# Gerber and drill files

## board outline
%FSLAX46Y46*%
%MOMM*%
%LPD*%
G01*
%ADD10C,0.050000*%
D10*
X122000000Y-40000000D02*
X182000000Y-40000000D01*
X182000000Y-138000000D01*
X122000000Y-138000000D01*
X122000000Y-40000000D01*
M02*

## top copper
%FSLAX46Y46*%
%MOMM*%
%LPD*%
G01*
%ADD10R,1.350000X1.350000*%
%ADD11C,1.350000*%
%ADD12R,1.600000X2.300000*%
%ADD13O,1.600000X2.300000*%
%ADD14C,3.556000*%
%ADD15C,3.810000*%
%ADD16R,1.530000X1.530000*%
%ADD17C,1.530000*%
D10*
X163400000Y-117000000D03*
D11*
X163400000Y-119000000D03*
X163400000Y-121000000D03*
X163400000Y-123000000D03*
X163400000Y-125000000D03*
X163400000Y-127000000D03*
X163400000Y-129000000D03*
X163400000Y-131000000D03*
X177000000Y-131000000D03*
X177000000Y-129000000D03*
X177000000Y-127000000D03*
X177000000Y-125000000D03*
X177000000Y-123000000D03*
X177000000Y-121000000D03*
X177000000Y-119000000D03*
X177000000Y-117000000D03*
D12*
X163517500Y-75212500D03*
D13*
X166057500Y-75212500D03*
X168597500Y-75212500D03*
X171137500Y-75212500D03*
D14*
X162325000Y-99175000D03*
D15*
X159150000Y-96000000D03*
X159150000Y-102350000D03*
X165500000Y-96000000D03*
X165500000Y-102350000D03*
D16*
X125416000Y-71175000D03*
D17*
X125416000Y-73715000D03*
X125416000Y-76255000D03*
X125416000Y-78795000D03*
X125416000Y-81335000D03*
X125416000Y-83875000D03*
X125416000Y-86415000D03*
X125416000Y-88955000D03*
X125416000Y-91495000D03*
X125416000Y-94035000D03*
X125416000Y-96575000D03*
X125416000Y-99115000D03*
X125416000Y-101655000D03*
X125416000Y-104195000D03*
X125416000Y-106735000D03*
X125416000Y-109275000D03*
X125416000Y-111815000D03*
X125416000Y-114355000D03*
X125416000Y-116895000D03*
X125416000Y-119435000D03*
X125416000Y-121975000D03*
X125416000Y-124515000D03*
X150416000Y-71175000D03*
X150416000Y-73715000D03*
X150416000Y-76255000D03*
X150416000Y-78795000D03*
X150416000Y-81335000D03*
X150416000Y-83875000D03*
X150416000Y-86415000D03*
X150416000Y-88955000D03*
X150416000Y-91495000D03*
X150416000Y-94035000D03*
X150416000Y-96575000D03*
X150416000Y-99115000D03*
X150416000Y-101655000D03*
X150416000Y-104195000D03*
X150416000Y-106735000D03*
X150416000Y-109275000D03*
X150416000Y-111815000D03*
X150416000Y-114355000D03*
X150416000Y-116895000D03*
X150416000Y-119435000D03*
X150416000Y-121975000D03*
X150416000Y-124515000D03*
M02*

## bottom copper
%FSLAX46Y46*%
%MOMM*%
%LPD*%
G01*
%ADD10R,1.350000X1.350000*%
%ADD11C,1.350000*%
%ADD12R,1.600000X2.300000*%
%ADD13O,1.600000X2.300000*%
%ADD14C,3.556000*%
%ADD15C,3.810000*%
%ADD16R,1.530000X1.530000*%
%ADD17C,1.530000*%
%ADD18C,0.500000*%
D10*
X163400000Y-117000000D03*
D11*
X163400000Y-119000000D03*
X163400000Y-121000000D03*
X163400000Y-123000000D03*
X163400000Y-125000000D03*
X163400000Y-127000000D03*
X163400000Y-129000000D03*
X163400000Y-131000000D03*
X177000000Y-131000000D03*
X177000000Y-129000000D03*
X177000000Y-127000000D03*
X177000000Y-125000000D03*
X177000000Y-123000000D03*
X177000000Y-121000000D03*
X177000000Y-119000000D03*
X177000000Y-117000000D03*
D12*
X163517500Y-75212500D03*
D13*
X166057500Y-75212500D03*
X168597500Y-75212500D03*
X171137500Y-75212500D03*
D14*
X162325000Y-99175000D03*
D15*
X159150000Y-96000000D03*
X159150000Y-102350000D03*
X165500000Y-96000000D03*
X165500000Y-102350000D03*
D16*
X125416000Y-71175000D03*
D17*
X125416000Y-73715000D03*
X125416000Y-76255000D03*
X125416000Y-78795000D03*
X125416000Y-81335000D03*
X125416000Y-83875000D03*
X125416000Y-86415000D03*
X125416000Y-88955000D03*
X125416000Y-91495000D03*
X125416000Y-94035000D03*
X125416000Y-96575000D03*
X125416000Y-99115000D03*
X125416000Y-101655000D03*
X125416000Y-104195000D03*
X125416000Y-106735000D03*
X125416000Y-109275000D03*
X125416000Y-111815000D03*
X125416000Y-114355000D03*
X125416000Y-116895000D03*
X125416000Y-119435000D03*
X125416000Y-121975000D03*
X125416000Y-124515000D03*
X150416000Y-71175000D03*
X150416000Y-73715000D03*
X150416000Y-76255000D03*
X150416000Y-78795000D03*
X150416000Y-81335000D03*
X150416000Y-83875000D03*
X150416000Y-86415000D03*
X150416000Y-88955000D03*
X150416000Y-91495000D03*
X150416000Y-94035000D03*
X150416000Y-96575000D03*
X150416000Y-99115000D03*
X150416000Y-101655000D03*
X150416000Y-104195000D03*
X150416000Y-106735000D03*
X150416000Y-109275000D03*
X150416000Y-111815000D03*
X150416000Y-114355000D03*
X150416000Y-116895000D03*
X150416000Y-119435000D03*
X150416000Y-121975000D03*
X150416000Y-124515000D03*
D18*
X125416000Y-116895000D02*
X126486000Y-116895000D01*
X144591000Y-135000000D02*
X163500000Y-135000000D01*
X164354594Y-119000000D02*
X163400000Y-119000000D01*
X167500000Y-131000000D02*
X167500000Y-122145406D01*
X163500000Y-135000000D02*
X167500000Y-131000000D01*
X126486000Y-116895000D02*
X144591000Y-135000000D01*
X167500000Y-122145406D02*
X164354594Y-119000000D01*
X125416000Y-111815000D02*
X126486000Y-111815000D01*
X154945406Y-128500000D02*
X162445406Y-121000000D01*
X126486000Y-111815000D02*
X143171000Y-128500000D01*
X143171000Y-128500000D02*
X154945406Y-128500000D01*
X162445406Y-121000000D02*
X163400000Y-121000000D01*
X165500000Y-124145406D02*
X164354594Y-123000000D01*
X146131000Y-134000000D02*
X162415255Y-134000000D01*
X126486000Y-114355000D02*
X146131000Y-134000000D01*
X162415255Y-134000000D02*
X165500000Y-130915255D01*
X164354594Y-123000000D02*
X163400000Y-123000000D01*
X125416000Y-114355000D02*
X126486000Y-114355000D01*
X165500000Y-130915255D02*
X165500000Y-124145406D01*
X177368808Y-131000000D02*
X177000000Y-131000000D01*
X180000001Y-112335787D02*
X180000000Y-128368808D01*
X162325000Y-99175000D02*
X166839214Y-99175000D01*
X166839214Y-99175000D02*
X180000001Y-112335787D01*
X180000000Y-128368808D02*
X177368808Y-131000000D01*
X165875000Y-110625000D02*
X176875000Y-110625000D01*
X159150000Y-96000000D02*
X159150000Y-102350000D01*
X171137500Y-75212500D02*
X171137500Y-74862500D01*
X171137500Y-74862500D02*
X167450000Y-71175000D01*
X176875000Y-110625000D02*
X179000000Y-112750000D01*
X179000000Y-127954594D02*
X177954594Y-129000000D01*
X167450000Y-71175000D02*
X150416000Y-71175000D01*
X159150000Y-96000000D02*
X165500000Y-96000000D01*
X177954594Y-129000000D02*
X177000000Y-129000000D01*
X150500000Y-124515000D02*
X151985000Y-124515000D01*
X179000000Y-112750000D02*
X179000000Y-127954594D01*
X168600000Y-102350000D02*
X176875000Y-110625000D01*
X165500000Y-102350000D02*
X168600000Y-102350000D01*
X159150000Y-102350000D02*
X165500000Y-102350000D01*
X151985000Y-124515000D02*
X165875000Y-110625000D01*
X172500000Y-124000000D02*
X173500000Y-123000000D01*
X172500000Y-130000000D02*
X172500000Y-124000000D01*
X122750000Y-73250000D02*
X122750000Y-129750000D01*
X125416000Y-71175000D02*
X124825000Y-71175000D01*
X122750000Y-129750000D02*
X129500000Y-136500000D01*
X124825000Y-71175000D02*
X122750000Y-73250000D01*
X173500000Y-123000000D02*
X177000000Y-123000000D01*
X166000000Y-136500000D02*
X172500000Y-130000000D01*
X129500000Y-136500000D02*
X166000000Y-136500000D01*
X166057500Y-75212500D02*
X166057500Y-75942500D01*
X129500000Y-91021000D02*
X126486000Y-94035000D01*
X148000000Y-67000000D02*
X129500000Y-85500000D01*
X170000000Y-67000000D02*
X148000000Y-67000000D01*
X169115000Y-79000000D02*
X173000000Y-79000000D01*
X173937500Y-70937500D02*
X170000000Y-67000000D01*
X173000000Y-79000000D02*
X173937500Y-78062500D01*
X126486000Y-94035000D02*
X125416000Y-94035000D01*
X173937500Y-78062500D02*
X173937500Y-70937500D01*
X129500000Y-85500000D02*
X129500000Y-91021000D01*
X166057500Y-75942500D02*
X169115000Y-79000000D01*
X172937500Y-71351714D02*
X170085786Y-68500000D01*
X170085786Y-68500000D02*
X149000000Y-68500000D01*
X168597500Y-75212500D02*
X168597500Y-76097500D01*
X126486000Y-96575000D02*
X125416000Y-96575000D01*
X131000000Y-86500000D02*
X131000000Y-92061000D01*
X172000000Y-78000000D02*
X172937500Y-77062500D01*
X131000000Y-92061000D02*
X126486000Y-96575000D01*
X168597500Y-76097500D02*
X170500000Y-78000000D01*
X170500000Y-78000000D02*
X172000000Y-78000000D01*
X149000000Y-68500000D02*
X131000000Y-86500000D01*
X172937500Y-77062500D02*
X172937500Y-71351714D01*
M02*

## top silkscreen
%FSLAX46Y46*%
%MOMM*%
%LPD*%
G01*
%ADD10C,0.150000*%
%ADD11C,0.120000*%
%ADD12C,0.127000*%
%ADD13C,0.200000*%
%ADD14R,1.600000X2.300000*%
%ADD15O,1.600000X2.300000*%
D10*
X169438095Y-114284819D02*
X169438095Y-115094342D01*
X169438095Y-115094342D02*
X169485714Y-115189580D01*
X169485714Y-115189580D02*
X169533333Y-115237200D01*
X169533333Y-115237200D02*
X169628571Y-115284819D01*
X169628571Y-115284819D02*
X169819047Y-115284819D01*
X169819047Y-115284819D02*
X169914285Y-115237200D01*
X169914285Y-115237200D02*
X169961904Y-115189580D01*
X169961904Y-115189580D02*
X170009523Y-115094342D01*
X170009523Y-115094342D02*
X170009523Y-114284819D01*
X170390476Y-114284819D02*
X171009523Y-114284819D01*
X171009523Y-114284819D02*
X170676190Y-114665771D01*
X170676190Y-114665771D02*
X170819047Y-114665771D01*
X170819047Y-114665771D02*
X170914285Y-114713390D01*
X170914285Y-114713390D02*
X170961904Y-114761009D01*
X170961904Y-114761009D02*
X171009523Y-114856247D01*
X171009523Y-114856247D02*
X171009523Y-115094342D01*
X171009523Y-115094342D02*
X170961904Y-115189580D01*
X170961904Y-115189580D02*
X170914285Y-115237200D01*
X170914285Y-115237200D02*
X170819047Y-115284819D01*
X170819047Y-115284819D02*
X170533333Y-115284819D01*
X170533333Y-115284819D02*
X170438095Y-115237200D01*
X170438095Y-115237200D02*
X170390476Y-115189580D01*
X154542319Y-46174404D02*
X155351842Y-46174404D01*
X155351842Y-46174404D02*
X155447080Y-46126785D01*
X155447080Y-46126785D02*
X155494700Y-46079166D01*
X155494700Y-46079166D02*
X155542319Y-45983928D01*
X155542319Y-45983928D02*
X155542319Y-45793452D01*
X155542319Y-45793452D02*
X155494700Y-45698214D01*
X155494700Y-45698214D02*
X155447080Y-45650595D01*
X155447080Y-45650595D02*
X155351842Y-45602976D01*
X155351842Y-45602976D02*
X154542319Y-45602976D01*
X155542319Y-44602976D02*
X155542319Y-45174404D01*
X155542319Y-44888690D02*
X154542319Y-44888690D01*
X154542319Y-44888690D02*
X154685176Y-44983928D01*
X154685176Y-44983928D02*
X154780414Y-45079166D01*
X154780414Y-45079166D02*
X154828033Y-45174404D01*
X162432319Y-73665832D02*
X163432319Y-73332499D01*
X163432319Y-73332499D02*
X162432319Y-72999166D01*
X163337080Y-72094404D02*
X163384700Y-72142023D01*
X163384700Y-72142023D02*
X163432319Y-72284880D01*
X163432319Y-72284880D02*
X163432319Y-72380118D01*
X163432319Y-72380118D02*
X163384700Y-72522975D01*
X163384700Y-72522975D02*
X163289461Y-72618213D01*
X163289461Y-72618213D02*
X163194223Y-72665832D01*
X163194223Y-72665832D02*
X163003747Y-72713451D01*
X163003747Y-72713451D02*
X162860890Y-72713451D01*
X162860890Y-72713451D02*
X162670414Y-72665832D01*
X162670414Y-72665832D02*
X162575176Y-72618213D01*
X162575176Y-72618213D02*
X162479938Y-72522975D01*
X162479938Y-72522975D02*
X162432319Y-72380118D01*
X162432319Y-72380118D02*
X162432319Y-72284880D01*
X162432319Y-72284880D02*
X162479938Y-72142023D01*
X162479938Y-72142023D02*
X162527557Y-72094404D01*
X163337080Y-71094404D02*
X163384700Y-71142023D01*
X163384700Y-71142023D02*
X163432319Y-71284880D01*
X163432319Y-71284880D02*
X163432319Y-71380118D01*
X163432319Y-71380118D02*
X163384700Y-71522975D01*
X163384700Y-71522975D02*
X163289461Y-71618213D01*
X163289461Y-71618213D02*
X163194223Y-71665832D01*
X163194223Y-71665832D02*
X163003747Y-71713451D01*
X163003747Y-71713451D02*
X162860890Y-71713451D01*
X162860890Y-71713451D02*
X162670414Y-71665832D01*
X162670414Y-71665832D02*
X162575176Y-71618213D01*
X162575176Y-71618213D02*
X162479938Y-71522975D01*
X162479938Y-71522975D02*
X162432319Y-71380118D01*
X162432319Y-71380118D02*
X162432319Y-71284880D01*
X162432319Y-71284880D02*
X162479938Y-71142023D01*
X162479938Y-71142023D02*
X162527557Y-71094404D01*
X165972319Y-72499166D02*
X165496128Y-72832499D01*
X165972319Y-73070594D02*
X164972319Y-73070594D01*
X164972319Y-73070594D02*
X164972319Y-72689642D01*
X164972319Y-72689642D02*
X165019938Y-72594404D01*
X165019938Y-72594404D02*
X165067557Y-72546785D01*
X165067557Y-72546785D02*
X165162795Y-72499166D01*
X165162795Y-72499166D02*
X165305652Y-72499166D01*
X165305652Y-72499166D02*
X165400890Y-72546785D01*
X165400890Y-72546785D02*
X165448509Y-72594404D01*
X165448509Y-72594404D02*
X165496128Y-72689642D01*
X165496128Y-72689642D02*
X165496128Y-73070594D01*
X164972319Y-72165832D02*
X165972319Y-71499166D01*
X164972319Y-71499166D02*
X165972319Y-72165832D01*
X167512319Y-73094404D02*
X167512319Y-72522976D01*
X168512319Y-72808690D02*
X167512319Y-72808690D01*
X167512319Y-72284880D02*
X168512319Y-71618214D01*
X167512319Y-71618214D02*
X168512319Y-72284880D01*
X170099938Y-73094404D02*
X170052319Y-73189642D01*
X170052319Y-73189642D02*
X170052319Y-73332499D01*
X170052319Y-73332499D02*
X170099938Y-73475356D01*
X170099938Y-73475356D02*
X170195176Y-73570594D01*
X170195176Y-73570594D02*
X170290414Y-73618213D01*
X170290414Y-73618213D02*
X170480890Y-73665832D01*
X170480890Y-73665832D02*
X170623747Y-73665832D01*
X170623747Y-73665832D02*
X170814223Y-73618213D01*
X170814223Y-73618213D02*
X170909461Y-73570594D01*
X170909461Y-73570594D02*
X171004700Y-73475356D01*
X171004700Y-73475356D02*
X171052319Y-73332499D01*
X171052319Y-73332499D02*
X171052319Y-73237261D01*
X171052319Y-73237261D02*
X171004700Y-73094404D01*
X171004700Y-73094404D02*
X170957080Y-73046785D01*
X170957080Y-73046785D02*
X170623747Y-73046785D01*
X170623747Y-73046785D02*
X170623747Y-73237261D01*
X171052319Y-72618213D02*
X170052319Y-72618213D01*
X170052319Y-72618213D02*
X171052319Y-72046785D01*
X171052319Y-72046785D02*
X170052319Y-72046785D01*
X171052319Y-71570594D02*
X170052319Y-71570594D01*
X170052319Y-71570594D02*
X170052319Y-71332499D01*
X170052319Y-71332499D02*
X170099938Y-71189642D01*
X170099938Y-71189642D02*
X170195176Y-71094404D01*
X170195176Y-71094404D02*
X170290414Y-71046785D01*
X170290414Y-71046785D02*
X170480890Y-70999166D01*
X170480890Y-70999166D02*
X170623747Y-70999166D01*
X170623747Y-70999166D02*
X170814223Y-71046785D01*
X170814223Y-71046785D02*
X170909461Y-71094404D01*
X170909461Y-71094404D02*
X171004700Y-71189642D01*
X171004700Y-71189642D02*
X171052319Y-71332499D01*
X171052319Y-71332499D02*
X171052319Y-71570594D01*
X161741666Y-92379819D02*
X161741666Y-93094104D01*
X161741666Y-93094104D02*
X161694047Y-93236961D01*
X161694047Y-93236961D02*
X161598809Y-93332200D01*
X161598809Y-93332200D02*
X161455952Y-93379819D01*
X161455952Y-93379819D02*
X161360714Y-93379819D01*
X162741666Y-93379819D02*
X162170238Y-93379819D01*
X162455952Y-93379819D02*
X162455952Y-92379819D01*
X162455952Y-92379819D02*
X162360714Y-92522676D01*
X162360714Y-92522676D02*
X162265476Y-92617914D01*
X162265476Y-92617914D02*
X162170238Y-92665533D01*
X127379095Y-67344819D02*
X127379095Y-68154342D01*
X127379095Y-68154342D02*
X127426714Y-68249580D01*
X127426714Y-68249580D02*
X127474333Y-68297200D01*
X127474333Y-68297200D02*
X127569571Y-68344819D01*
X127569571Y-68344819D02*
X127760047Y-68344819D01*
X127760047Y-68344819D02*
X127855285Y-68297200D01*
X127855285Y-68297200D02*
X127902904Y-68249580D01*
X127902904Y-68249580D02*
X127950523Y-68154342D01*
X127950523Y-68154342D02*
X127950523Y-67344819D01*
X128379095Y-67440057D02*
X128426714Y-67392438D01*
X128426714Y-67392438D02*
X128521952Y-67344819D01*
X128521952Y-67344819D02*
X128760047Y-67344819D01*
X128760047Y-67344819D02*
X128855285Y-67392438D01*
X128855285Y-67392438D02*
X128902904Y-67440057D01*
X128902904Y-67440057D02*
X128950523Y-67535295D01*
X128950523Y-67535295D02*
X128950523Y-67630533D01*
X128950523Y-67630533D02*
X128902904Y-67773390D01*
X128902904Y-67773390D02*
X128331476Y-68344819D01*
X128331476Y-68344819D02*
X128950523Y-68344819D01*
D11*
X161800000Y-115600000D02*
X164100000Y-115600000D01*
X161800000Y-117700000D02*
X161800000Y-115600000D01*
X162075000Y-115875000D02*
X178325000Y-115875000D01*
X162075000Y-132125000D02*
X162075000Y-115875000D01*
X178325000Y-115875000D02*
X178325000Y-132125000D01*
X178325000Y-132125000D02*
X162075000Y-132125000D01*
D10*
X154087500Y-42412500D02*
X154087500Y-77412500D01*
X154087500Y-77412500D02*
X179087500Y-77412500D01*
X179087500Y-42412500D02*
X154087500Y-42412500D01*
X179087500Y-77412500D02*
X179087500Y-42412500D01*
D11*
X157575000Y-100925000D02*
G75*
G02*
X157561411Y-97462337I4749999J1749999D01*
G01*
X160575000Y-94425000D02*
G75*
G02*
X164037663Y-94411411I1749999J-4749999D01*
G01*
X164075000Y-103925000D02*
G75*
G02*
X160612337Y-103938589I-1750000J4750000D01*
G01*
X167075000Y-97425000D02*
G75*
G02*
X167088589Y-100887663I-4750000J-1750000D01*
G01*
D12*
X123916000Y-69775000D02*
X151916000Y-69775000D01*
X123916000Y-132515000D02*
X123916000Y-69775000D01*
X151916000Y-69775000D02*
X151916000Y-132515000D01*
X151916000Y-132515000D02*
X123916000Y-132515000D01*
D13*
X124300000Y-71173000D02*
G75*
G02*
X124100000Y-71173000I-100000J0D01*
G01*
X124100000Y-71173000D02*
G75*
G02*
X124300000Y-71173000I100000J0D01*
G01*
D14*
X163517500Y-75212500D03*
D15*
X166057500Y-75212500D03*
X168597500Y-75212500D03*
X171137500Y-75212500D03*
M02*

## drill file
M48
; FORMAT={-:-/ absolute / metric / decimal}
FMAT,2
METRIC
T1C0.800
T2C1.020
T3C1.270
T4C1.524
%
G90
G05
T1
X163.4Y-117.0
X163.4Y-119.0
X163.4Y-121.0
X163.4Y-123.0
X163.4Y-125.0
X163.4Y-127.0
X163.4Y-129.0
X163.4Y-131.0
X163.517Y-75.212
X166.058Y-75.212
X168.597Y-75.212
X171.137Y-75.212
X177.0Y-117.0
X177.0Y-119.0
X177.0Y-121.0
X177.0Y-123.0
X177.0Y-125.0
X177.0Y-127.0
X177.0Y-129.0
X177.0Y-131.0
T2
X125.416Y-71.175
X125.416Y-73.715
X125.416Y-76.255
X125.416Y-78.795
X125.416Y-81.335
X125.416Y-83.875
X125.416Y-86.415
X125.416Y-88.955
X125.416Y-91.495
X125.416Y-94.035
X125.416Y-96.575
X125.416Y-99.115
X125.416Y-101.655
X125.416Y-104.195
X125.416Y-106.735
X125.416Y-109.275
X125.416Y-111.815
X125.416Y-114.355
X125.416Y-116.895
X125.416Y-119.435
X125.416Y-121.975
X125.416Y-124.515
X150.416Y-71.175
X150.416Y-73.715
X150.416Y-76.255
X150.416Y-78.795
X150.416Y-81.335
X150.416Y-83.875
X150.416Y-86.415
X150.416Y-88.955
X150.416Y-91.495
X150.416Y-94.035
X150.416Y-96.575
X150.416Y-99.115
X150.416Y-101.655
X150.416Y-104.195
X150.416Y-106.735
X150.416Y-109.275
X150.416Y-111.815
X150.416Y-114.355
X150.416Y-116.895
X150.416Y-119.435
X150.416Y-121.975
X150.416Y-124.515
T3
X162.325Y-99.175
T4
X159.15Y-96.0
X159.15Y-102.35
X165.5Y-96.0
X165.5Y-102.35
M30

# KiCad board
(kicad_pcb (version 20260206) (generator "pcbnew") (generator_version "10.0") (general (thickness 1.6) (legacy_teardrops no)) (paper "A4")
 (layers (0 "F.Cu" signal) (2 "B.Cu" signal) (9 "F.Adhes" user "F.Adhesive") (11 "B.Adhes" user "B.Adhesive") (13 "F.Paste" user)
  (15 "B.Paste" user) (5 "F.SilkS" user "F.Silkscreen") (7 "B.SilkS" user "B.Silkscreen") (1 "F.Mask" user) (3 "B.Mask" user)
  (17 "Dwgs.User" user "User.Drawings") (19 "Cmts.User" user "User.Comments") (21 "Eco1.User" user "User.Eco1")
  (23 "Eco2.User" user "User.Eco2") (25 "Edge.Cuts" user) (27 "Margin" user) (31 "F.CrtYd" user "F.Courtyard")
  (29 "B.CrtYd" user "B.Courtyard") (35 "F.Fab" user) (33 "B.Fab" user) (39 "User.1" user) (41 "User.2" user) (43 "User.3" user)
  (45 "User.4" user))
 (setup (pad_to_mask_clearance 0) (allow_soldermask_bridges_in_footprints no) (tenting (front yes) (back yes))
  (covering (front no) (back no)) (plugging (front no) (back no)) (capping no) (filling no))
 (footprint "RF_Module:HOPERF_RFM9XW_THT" (layer "F.Cu") (at 163.4 117)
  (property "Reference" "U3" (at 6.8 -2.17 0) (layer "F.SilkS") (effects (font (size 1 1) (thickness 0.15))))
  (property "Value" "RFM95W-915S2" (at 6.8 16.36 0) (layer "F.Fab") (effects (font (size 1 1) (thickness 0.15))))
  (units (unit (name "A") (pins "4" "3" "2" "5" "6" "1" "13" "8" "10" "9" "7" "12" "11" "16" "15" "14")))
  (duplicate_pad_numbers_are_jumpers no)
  (fp_line (start -1.6 -1.4) (end 0.7 -1.4) (stroke (width 0.12) (type solid)) (layer "F.SilkS"))
  (fp_line (start -1.6 0.7) (end -1.6 -1.4) (stroke (width 0.12) (type solid)) (layer "F.SilkS"))
  (fp_line (start -1.325 -1.125) (end 14.925 -1.125) (stroke (width 0.12) (type solid)) (layer "F.SilkS"))
  (fp_line (start -1.325 15.125) (end -1.325 -1.125) (stroke (width 0.12) (type solid)) (layer "F.SilkS"))
  (fp_line (start 14.925 -1.125) (end 14.925 15.125) (stroke (width 0.12) (type solid)) (layer "F.SilkS"))
  (fp_line (start 14.925 15.125) (end -1.325 15.125) (stroke (width 0.12) (type solid)) (layer "F.SilkS"))
  (pad "1" thru_hole rect (at 0 0) (size 1.35 1.35) (drill 0.8) (layers "*.Cu" "*.Mask") (remove_unused_layers no)
   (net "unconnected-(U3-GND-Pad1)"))
  (pad "2" thru_hole circle (at 0 2) (size 1.35 1.35) (drill 0.8) (layers "*.Cu" "*.Mask") (remove_unused_layers no) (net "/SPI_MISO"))
  (pad "3" thru_hole circle (at 0 4) (size 1.35 1.35) (drill 0.8) (layers "*.Cu" "*.Mask") (remove_unused_layers no) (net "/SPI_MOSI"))
  (pad "4" thru_hole circle (at 0 6) (size 1.35 1.35) (drill 0.8) (layers "*.Cu" "*.Mask") (remove_unused_layers no) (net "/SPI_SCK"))
  (pad "5" thru_hole circle (at 0 8) (size 1.35 1.35) (drill 0.8) (layers "*.Cu" "*.Mask") (remove_unused_layers no) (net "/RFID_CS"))
  (pad "6" thru_hole circle (at 0 10) (size 1.35 1.35) (drill 0.8) (layers "*.Cu" "*.Mask") (remove_unused_layers no) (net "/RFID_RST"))
  (pad "7" thru_hole circle (at 0 12) (size 1.35 1.35) (drill 0.8) (layers "*.Cu" "*.Mask") (remove_unused_layers no)
   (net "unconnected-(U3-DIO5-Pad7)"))
  (pad "8" thru_hole circle (at 0 14) (size 1.35 1.35) (drill 0.8) (layers "*.Cu" "*.Mask") (remove_unused_layers no)
   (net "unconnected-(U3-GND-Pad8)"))
  (pad "9" thru_hole circle (at 13.6 14) (size 1.35 1.35) (drill 0.8) (layers "*.Cu" "*.Mask") (remove_unused_layers no) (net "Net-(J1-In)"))
  (pad "10" thru_hole circle (at 13.6 12) (size 1.35 1.35) (drill 0.8) (layers "*.Cu" "*.Mask") (remove_unused_layers no)
   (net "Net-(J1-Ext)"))
  (pad "11" thru_hole circle (at 13.6 10) (size 1.35 1.35) (drill 0.8) (layers "*.Cu" "*.Mask") (remove_unused_layers no)
   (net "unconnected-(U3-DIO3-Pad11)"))
  (pad "12" thru_hole circle (at 13.6 8) (size 1.35 1.35) (drill 0.8) (layers "*.Cu" "*.Mask") (remove_unused_layers no)
   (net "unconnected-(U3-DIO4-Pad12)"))
  (pad "13" thru_hole circle (at 13.6 6) (size 1.35 1.35) (drill 0.8) (layers "*.Cu" "*.Mask") (remove_unused_layers no)
   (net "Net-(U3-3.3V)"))
  (pad "14" thru_hole circle (at 13.6 4) (size 1.35 1.35) (drill 0.8) (layers "*.Cu" "*.Mask") (remove_unused_layers no)
   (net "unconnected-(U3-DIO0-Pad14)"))
  (pad "15" thru_hole circle (at 13.6 2) (size 1.35 1.35) (drill 0.8) (layers "*.Cu" "*.Mask") (remove_unused_layers no)
   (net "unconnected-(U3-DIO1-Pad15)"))
  (pad "16" thru_hole circle (at 13.6 0) (size 1.35 1.35) (drill 0.8) (layers "*.Cu" "*.Mask") (remove_unused_layers no)
   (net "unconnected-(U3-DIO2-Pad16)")))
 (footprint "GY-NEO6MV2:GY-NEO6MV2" (layer "F.Cu") (at 154.0875 77.4125 -90)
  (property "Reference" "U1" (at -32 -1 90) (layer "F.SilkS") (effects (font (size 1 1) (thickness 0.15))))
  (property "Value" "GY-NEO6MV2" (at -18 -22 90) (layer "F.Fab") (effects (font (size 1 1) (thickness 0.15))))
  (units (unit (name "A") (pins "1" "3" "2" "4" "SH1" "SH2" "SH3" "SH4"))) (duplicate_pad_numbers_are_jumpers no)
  (fp_line (start -35 0) (end 0 0) (stroke (width 0.15) (type solid)) (layer "F.SilkS"))
  (fp_line (start 0 0) (end 0 -25) (stroke (width 0.15) (type solid)) (layer "F.SilkS"))
  (fp_line (start -35 -25) (end -35 0) (stroke (width 0.15) (type solid)) (layer "F.SilkS"))
  (fp_line (start 0 -25) (end -35 -25) (stroke (width 0.15) (type solid)) (layer "F.SilkS"))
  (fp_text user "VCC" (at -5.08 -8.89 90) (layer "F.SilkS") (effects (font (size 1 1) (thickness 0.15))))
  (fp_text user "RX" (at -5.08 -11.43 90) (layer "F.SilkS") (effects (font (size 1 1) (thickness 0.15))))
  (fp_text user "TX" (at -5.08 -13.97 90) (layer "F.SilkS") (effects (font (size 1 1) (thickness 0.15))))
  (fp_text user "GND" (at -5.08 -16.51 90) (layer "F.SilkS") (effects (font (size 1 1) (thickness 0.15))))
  (pad "1" thru_hole rect (at -2.2 -9.43 270) (size 2.3 1.6) (drill 0.8) (layers "*.Cu" "*.Mask" "F.SilkS") (remove_unused_layers no)
   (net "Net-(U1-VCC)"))
  (pad "2" thru_hole oval (at -2.2 -11.97 270) (size 2.3 1.6) (drill 0.8) (layers "*.Cu" "*.Mask" "F.SilkS") (remove_unused_layers no)
   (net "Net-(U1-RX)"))
  (pad "3" thru_hole oval (at -2.2 -14.51 270) (size 2.3 1.6) (drill 0.8) (layers "*.Cu" "*.Mask" "F.SilkS") (remove_unused_layers no)
   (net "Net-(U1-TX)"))
  (pad "4" thru_hole oval (at -2.2 -17.05 270) (size 2.3 1.6) (drill 0.8) (layers "*.Cu" "*.Mask" "F.SilkS") (remove_unused_layers no)
   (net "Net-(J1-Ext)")))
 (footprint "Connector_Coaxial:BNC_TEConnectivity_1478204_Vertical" (layer "F.Cu") (at 162.325 99.175)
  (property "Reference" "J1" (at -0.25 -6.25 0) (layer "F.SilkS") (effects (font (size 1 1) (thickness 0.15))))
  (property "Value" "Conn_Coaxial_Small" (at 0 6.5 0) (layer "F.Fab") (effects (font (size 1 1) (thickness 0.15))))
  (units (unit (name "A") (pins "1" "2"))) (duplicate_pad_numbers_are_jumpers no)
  (fp_arc (start -4.75 1.75) (mid -5.062075 0.019867) (end -4.763589 -1.712663) (stroke (width 0.12) (type solid)) (layer "F.SilkS"))
  (fp_arc (start -1.75 -4.75) (mid -0.019867 -5.062075) (end 1.712663 -4.763589) (stroke (width 0.12) (type solid)) (layer "F.SilkS"))
  (fp_arc (start 1.75 4.75) (mid 0.019867 5.062075) (end -1.712663 4.763589) (stroke (width 0.12) (type solid)) (layer "F.SilkS"))
  (fp_arc (start 4.75 -1.75) (mid 5.062075 -0.019867) (end 4.763589 1.712663) (stroke (width 0.12) (type solid)) (layer "F.SilkS"))
  (pad "1" thru_hole circle (at 0 0) (size 3.556 3.556) (drill 1.27) (layers "*.Cu" "*.Mask") (remove_unused_layers no) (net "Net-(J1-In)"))
  (pad "2" thru_hole circle (at -3.175 -3.175) (size 3.81 3.81) (drill 1.524) (layers "*.Cu" "*.Mask") (remove_unused_layers no)
   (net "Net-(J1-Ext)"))
  (pad "2" thru_hole circle (at -3.175 3.175) (size 3.81 3.81) (drill 1.524) (layers "*.Cu" "*.Mask") (remove_unused_layers no)
   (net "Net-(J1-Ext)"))
  (pad "2" thru_hole circle (at 3.175 -3.175) (size 3.81 3.81) (drill 1.524) (layers "*.Cu" "*.Mask") (remove_unused_layers no)
   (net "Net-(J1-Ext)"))
  (pad "2" thru_hole circle (at 3.175 3.175) (size 3.81 3.81) (drill 1.524) (layers "*.Cu" "*.Mask") (remove_unused_layers no)
   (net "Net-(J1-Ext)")))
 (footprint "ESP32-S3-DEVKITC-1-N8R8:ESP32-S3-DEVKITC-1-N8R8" (layer "F.Cu") (at 137.916 101.145)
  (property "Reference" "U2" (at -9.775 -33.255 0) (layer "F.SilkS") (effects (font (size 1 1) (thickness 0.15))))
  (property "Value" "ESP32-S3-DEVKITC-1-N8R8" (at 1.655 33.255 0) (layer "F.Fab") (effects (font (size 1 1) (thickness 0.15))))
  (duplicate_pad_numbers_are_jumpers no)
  (fp_line (start -14 -31.37) (end 14 -31.37) (stroke (width 0.127) (type solid)) (layer "F.SilkS"))
  (fp_line (start -14 31.37) (end -14 -31.37) (stroke (width 0.127) (type solid)) (layer "F.SilkS"))
  (fp_line (start 14 -31.37) (end 14 31.37) (stroke (width 0.127) (type solid)) (layer "F.SilkS"))
  (fp_line (start 14 31.37) (end -14 31.37) (stroke (width 0.127) (type solid)) (layer "F.SilkS"))
  (fp_circle (center -13.716 -29.972) (end -13.616 -29.972) (stroke (width 0.2) (type solid)) (fill no) (layer "F.SilkS"))
  (pad "J1_1" thru_hole rect (at -12.5 -29.97) (size 1.53 1.53) (drill 1.02) (layers "*.Cu" "*.Mask") (remove_unused_layers no)
   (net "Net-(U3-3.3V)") (solder_mask_margin 0.102))
  (pad "J1_2" thru_hole circle (at -12.5 -27.43) (size 1.53 1.53) (drill 1.02) (layers "*.Cu" "*.Mask") (remove_unused_layers no)
   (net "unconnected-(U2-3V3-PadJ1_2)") (solder_mask_margin 0.102))
  (pad "J1_3" thru_hole circle (at -12.5 -24.89) (size 1.53 1.53) (drill 1.02) (layers "*.Cu" "*.Mask") (remove_unused_layers no)
   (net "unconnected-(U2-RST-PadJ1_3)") (solder_mask_margin 0.102))
  (pad "J1_4" thru_hole circle (at -12.5 -22.35) (size 1.53 1.53) (drill 1.02) (layers "*.Cu" "*.Mask") (remove_unused_layers no)
   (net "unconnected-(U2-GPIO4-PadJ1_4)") (solder_mask_margin 0.102))
  (pad "J1_5" thru_hole circle (at -12.5 -19.81) (size 1.53 1.53) (drill 1.02) (layers "*.Cu" "*.Mask") (remove_unused_layers no)
   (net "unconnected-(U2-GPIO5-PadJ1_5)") (solder_mask_margin 0.102))
  (pad "J1_6" thru_hole circle (at -12.5 -17.27) (size 1.53 1.53) (drill 1.02) (layers "*.Cu" "*.Mask") (remove_unused_layers no)
   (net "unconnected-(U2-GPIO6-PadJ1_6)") (solder_mask_margin 0.102))
  (pad "J1_7" thru_hole circle (at -12.5 -14.73) (size 1.53 1.53) (drill 1.02) (layers "*.Cu" "*.Mask") (remove_unused_layers no)
   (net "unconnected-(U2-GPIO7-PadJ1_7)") (solder_mask_margin 0.102))
  (pad "J1_8" thru_hole circle (at -12.5 -12.19) (size 1.53 1.53) (drill 1.02) (layers "*.Cu" "*.Mask") (remove_unused_layers no)
   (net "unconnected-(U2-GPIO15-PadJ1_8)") (solder_mask_margin 0.102))
  (pad "J1_9" thru_hole circle (at -12.5 -9.65) (size 1.53 1.53) (drill 1.02) (layers "*.Cu" "*.Mask") (remove_unused_layers no)
   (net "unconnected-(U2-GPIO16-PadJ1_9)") (solder_mask_margin 0.102))
  (pad "J1_10" thru_hole circle (at -12.5 -7.11) (size 1.53 1.53) (drill 1.02) (layers "*.Cu" "*.Mask") (remove_unused_layers no)
   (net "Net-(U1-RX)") (solder_mask_margin 0.102))
  (pad "J1_11" thru_hole circle (at -12.5 -4.57) (size 1.53 1.53) (drill 1.02) (layers "*.Cu" "*.Mask") (remove_unused_layers no)
   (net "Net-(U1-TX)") (solder_mask_margin 0.102))
  (pad "J1_12" thru_hole circle (at -12.5 -2.03) (size 1.53 1.53) (drill 1.02) (layers "*.Cu" "*.Mask") (remove_unused_layers no)
   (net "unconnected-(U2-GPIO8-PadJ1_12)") (solder_mask_margin 0.102))
  (pad "J1_13" thru_hole circle (at -12.5 0.51) (size 1.53 1.53) (drill 1.02) (layers "*.Cu" "*.Mask") (remove_unused_layers no)
   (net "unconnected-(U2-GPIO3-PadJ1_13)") (solder_mask_margin 0.102))
  (pad "J1_14" thru_hole circle (at -12.5 3.05) (size 1.53 1.53) (drill 1.02) (layers "*.Cu" "*.Mask") (remove_unused_layers no)
   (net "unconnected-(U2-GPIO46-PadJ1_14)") (solder_mask_margin 0.102))
  (pad "J1_15" thru_hole circle (at -12.5 5.59) (size 1.53 1.53) (drill 1.02) (layers "*.Cu" "*.Mask") (remove_unused_layers no)
   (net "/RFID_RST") (solder_mask_margin 0.102))
  (pad "J1_16" thru_hole circle (at -12.5 8.13) (size 1.53 1.53) (drill 1.02) (layers "*.Cu" "*.Mask") (remove_unused_layers no)
   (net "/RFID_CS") (solder_mask_margin 0.102))
  (pad "J1_17" thru_hole circle (at -12.5 10.67) (size 1.53 1.53) (drill 1.02) (layers "*.Cu" "*.Mask") (remove_unused_layers no)
   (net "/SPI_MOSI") (solder_mask_margin 0.102))
  (pad "J1_18" thru_hole circle (at -12.5 13.21) (size 1.53 1.53) (drill 1.02) (layers "*.Cu" "*.Mask") (remove_unused_layers no)
   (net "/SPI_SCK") (solder_mask_margin 0.102))
  (pad "J1_19" thru_hole circle (at -12.5 15.75) (size 1.53 1.53) (drill 1.02) (layers "*.Cu" "*.Mask") (remove_unused_layers no)
   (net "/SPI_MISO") (solder_mask_margin 0.102))
  (pad "J1_20" thru_hole circle (at -12.5 18.29) (size 1.53 1.53) (drill 1.02) (layers "*.Cu" "*.Mask") (remove_unused_layers no)
   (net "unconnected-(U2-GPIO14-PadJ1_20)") (solder_mask_margin 0.102))
  (pad "J1_21" thru_hole circle (at -12.5 20.83) (size 1.53 1.53) (drill 1.02) (layers "*.Cu" "*.Mask") (remove_unused_layers no)
   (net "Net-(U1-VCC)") (solder_mask_margin 0.102))
  (pad "J1_22" thru_hole circle (at -12.5 23.37) (size 1.53 1.53) (drill 1.02) (layers "*.Cu" "*.Mask") (remove_unused_layers no)
   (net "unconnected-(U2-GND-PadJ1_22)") (solder_mask_margin 0.102))
  (pad "J3_1" thru_hole circle (at 12.5 -29.97) (size 1.53 1.53) (drill 1.02) (layers "*.Cu" "*.Mask") (remove_unused_layers no)
   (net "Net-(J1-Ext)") (solder_mask_margin 0.102))
  (pad "J3_2" thru_hole circle (at 12.5 -27.43) (size 1.53 1.53) (drill 1.02) (layers "*.Cu" "*.Mask") (remove_unused_layers no)
   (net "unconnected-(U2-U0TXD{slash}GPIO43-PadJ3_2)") (solder_mask_margin 0.102))
  (pad "J3_3" thru_hole circle (at 12.5 -24.89) (size 1.53 1.53) (drill 1.02) (layers "*.Cu" "*.Mask") (remove_unused_layers no)
   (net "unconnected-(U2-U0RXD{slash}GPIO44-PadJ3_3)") (solder_mask_margin 0.102))
  (pad "J3_4" thru_hole circle (at 12.5 -22.35) (size 1.53 1.53) (drill 1.02) (layers "*.Cu" "*.Mask") (remove_unused_layers no)
   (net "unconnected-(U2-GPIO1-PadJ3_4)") (solder_mask_margin 0.102))
  (pad "J3_5" thru_hole circle (at 12.5 -19.81) (size 1.53 1.53) (drill 1.02) (layers "*.Cu" "*.Mask") (remove_unused_layers no)
   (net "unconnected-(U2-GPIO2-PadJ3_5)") (solder_mask_margin 0.102))
  (pad "J3_6" thru_hole circle (at 12.5 -17.27) (size 1.53 1.53) (drill 1.02) (layers "*.Cu" "*.Mask") (remove_unused_layers no)
   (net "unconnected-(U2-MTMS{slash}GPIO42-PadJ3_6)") (solder_mask_margin 0.102))
  (pad "J3_7" thru_hole circle (at 12.5 -14.73) (size 1.53 1.53) (drill 1.02) (layers "*.Cu" "*.Mask") (remove_unused_layers no)
   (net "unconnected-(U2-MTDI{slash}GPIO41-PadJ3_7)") (solder_mask_margin 0.102))
  (pad "J3_8" thru_hole circle (at 12.5 -12.19) (size 1.53 1.53) (drill 1.02) (layers "*.Cu" "*.Mask") (remove_unused_layers no)
   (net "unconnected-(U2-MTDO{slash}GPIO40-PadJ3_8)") (solder_mask_margin 0.102))
  (pad "J3_9" thru_hole circle (at 12.5 -9.65) (size 1.53 1.53) (drill 1.02) (layers "*.Cu" "*.Mask") (remove_unused_layers no)
   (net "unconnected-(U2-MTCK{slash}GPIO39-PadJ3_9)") (solder_mask_margin 0.102))
  (pad "J3_10" thru_hole circle (at 12.5 -7.11) (size 1.53 1.53) (drill 1.02) (layers "*.Cu" "*.Mask") (remove_unused_layers no)
   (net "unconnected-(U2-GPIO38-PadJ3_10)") (solder_mask_margin 0.102))
  (pad "J3_11" thru_hole circle (at 12.5 -4.57) (size 1.53 1.53) (drill 1.02) (layers "*.Cu" "*.Mask") (remove_unused_layers no)
   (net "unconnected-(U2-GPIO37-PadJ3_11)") (solder_mask_margin 0.102))
  (pad "J3_12" thru_hole circle (at 12.5 -2.03) (size 1.53 1.53) (drill 1.02) (layers "*.Cu" "*.Mask") (remove_unused_layers no)
   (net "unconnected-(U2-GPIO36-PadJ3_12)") (solder_mask_margin 0.102))
  (pad "J3_13" thru_hole circle (at 12.5 0.51) (size 1.53 1.53) (drill 1.02) (layers "*.Cu" "*.Mask") (remove_unused_layers no)
   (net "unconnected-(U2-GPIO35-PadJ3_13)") (solder_mask_margin 0.102))
  (pad "J3_14" thru_hole circle (at 12.5 3.05) (size 1.53 1.53) (drill 1.02) (layers "*.Cu" "*.Mask") (remove_unused_layers no)
   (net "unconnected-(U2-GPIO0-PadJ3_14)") (solder_mask_margin 0.102))
  (pad "J3_15" thru_hole circle (at 12.5 5.59) (size 1.53 1.53) (drill 1.02) (layers "*.Cu" "*.Mask") (remove_unused_layers no)
   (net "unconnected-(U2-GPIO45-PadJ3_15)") (solder_mask_margin 0.102))
  (pad "J3_16" thru_hole circle (at 12.5 8.13) (size 1.53 1.53) (drill 1.02) (layers "*.Cu" "*.Mask") (remove_unused_layers no)
   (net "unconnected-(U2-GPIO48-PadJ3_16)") (solder_mask_margin 0.102))
  (pad "J3_17" thru_hole circle (at 12.5 10.67) (size 1.53 1.53) (drill 1.02) (layers "*.Cu" "*.Mask") (remove_unused_layers no)
   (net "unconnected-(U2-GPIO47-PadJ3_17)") (solder_mask_margin 0.102))
  (pad "J3_18" thru_hole circle (at 12.5 13.21) (size 1.53 1.53) (drill 1.02) (layers "*.Cu" "*.Mask") (remove_unused_layers no)
   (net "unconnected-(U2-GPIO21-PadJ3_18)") (solder_mask_margin 0.102))
  (pad "J3_19" thru_hole circle (at 12.5 15.75) (size 1.53 1.53) (drill 1.02) (layers "*.Cu" "*.Mask") (remove_unused_layers no)
   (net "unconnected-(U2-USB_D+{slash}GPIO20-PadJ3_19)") (solder_mask_margin 0.102))
  (pad "J3_20" thru_hole circle (at 12.5 18.29) (size 1.53 1.53) (drill 1.02) (layers "*.Cu" "*.Mask") (remove_unused_layers no)
   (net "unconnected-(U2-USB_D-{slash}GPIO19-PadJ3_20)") (solder_mask_margin 0.102))
  (pad "J3_21" thru_hole circle (at 12.5 20.83) (size 1.53 1.53) (drill 1.02) (layers "*.Cu" "*.Mask") (remove_unused_layers no)
   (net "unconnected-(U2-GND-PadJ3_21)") (solder_mask_margin 0.102))
  (pad "J3_22" thru_hole circle (at 12.5 23.37) (size 1.53 1.53) (drill 1.02) (layers "*.Cu" "*.Mask") (remove_unused_layers no)
   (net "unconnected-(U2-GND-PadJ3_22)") (solder_mask_margin 0.102)))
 (gr_rect (start 122 40) (end 182 138) (stroke (width 0.05) (type solid)) (fill no) (layer "Edge.Cuts"))
 (segment (start 125.416 116.895) (end 126.486 116.895) (width 0.5) (layer "B.Cu") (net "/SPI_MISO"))
 (segment (start 144.591 135) (end 163.5 135) (width 0.5) (layer "B.Cu") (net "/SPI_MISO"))
 (segment (start 164.354594 119) (end 163.4 119) (width 0.5) (layer "B.Cu") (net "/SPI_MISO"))
 (segment (start 167.5 131) (end 167.5 122.145406) (width 0.5) (layer "B.Cu") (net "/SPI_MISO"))
 (segment (start 163.5 135) (end 167.5 131) (width 0.5) (layer "B.Cu") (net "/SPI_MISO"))
 (segment (start 126.486 116.895) (end 144.591 135) (width 0.5) (layer "B.Cu") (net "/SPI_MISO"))
 (segment (start 167.5 122.145406) (end 164.354594 119) (width 0.5) (layer "B.Cu") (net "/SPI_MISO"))
 (segment (start 125.416 111.815) (end 126.486 111.815) (width 0.5) (layer "B.Cu") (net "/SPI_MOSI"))
 (segment (start 154.945406 128.5) (end 162.445406 121) (width 0.5) (layer "B.Cu") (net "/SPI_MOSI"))
 (segment (start 126.486 111.815) (end 143.171 128.5) (width 0.5) (layer "B.Cu") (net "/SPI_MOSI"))
 (segment (start 143.171 128.5) (end 154.945406 128.5) (width 0.5) (layer "B.Cu") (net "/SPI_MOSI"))
 (segment (start 162.445406 121) (end 163.4 121) (width 0.5) (layer "B.Cu") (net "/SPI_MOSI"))
 (segment (start 165.5 124.145406) (end 164.354594 123) (width 0.5) (layer "B.Cu") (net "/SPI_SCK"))
 (segment (start 146.131 134) (end 162.415255 134) (width 0.5) (layer "B.Cu") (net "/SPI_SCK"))
 (segment (start 126.486 114.355) (end 146.131 134) (width 0.5) (layer "B.Cu") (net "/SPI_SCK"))
 (segment (start 162.415255 134) (end 165.5 130.915255) (width 0.5) (layer "B.Cu") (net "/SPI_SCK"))
 (segment (start 164.354594 123) (end 163.4 123) (width 0.5) (layer "B.Cu") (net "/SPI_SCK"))
 (segment (start 125.416 114.355) (end 126.486 114.355) (width 0.5) (layer "B.Cu") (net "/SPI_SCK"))
 (segment (start 165.5 130.915255) (end 165.5 124.145406) (width 0.5) (layer "B.Cu") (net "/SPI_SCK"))
 (segment (start 177.368808 131) (end 177 131) (width 0.5) (layer "B.Cu") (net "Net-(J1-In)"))
 (segment (start 180.000001 112.335787) (end 180 128.368808) (width 0.5) (layer "B.Cu") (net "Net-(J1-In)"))
 (segment (start 162.325 99.175) (end 166.839214 99.175) (width 0.5) (layer "B.Cu") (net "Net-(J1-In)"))
 (segment (start 166.839214 99.175) (end 180.000001 112.335787) (width 0.5) (layer "B.Cu") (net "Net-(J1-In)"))
 (segment (start 180 128.368808) (end 177.368808 131) (width 0.5) (layer "B.Cu") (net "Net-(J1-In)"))
 (segment (start 165.875 110.625) (end 176.875 110.625) (width 0.5) (layer "B.Cu") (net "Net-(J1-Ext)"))
 (segment (start 159.15 96) (end 159.15 102.35) (width 0.5) (layer "B.Cu") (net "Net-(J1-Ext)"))
 (segment (start 171.1375 75.2125) (end 171.1375 74.8625) (width 0.5) (layer "B.Cu") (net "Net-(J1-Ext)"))
 (segment (start 171.1375 74.8625) (end 167.45 71.175) (width 0.5) (layer "B.Cu") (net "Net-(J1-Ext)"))
 (segment (start 176.875 110.625) (end 179 112.75) (width 0.5) (layer "B.Cu") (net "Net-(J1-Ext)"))
 (segment (start 179 127.954594) (end 177.954594 129) (width 0.5) (layer "B.Cu") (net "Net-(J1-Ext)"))
 (segment (start 167.45 71.175) (end 150.416 71.175) (width 0.5) (layer "B.Cu") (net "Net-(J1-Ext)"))
 (segment (start 159.15 96) (end 165.5 96) (width 0.5) (layer "B.Cu") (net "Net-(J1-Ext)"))
 (segment (start 177.954594 129) (end 177 129) (width 0.5) (layer "B.Cu") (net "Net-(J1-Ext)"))
 (segment (start 150.5 124.515) (end 151.985 124.515) (width 0.5) (layer "B.Cu") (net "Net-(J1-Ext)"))
 (segment (start 179 112.75) (end 179 127.954594) (width 0.5) (layer "B.Cu") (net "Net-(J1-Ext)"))
 (segment (start 168.6 102.35) (end 176.875 110.625) (width 0.5) (layer "B.Cu") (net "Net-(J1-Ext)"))
 (segment (start 165.5 102.35) (end 168.6 102.35) (width 0.5) (layer "B.Cu") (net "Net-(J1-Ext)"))
 (segment (start 159.15 102.35) (end 165.5 102.35) (width 0.5) (layer "B.Cu") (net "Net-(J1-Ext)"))
 (segment (start 151.985 124.515) (end 165.875 110.625) (width 0.5) (layer "B.Cu") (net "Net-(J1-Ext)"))
 (segment (start 172.5 124) (end 173.5 123) (width 0.5) (layer "B.Cu") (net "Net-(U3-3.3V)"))
 (segment (start 172.5 130) (end 172.5 124) (width 0.5) (layer "B.Cu") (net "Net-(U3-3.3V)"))
 (segment (start 122.75 73.25) (end 122.75 129.75) (width 0.5) (layer "B.Cu") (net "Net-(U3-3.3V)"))
 (segment (start 125.416 71.175) (end 124.825 71.175) (width 0.5) (layer "B.Cu") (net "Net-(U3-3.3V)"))
 (segment (start 122.75 129.75) (end 129.5 136.5) (width 0.5) (layer "B.Cu") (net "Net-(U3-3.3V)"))
 (segment (start 124.825 71.175) (end 122.75 73.25) (width 0.5) (layer "B.Cu") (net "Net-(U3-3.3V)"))
 (segment (start 173.5 123) (end 177 123) (width 0.5) (layer "B.Cu") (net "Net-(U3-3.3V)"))
 (segment (start 166 136.5) (end 172.5 130) (width 0.5) (layer "B.Cu") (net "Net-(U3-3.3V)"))
 (segment (start 129.5 136.5) (end 166 136.5) (width 0.5) (layer "B.Cu") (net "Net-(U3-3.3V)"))
 (segment (start 166.0575 75.2125) (end 166.0575 75.9425) (width 0.5) (layer "B.Cu") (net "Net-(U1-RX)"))
 (segment (start 129.5 91.021) (end 126.486 94.035) (width 0.5) (layer "B.Cu") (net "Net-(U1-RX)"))
 (segment (start 148 67) (end 129.5 85.5) (width 0.5) (layer "B.Cu") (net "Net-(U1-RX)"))
 (segment (start 170 67) (end 148 67) (width 0.5) (layer "B.Cu") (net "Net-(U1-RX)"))
 (segment (start 169.115 79) (end 173 79) (width 0.5) (layer "B.Cu") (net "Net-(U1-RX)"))
 (segment (start 173.9375 70.9375) (end 170 67) (width 0.5) (layer "B.Cu") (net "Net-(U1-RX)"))
 (segment (start 173 79) (end 173.9375 78.0625) (width 0.5) (layer "B.Cu") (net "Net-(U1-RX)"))
 (segment (start 126.486 94.035) (end 125.416 94.035) (width 0.5) (layer "B.Cu") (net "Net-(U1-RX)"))
 (segment (start 173.9375 78.0625) (end 173.9375 70.9375) (width 0.5) (layer "B.Cu") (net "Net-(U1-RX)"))
 (segment (start 129.5 85.5) (end 129.5 91.021) (width 0.5) (layer "B.Cu") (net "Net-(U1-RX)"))
 (segment (start 166.0575 75.9425) (end 169.115 79) (width 0.5) (layer "B.Cu") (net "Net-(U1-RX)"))
 (segment (start 172.9375 71.351714) (end 170.085786 68.5) (width 0.5) (layer "B.Cu") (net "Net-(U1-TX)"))
 (segment (start 170.085786 68.5) (end 149 68.5) (width 0.5) (layer "B.Cu") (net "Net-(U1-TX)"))
 (segment (start 168.5975 75.2125) (end 168.5975 76.0975) (width 0.5) (layer "B.Cu") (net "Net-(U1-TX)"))
 (segment (start 126.486 96.575) (end 125.416 96.575) (width 0.5) (layer "B.Cu") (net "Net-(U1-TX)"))
 (segment (start 131 86.5) (end 131 92.061) (width 0.5) (layer "B.Cu") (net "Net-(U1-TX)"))
 (segment (start 172 78) (end 172.9375 77.0625) (width 0.5) (layer "B.Cu") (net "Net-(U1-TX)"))
 (segment (start 131 92.061) (end 126.486 96.575) (width 0.5) (layer "B.Cu") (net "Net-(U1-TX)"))
 (segment (start 168.5975 76.0975) (end 170.5 78) (width 0.5) (layer "B.Cu") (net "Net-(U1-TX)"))
 (segment (start 170.5 78) (end 172 78) (width 0.5) (layer "B.Cu") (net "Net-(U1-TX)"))
 (segment (start 149 68.5) (end 131 86.5) (width 0.5) (layer "B.Cu") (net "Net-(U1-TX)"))
 (segment (start 172.9375 77.0625) (end 172.9375 71.351714) (width 0.5) (layer "B.Cu") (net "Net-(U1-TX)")))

